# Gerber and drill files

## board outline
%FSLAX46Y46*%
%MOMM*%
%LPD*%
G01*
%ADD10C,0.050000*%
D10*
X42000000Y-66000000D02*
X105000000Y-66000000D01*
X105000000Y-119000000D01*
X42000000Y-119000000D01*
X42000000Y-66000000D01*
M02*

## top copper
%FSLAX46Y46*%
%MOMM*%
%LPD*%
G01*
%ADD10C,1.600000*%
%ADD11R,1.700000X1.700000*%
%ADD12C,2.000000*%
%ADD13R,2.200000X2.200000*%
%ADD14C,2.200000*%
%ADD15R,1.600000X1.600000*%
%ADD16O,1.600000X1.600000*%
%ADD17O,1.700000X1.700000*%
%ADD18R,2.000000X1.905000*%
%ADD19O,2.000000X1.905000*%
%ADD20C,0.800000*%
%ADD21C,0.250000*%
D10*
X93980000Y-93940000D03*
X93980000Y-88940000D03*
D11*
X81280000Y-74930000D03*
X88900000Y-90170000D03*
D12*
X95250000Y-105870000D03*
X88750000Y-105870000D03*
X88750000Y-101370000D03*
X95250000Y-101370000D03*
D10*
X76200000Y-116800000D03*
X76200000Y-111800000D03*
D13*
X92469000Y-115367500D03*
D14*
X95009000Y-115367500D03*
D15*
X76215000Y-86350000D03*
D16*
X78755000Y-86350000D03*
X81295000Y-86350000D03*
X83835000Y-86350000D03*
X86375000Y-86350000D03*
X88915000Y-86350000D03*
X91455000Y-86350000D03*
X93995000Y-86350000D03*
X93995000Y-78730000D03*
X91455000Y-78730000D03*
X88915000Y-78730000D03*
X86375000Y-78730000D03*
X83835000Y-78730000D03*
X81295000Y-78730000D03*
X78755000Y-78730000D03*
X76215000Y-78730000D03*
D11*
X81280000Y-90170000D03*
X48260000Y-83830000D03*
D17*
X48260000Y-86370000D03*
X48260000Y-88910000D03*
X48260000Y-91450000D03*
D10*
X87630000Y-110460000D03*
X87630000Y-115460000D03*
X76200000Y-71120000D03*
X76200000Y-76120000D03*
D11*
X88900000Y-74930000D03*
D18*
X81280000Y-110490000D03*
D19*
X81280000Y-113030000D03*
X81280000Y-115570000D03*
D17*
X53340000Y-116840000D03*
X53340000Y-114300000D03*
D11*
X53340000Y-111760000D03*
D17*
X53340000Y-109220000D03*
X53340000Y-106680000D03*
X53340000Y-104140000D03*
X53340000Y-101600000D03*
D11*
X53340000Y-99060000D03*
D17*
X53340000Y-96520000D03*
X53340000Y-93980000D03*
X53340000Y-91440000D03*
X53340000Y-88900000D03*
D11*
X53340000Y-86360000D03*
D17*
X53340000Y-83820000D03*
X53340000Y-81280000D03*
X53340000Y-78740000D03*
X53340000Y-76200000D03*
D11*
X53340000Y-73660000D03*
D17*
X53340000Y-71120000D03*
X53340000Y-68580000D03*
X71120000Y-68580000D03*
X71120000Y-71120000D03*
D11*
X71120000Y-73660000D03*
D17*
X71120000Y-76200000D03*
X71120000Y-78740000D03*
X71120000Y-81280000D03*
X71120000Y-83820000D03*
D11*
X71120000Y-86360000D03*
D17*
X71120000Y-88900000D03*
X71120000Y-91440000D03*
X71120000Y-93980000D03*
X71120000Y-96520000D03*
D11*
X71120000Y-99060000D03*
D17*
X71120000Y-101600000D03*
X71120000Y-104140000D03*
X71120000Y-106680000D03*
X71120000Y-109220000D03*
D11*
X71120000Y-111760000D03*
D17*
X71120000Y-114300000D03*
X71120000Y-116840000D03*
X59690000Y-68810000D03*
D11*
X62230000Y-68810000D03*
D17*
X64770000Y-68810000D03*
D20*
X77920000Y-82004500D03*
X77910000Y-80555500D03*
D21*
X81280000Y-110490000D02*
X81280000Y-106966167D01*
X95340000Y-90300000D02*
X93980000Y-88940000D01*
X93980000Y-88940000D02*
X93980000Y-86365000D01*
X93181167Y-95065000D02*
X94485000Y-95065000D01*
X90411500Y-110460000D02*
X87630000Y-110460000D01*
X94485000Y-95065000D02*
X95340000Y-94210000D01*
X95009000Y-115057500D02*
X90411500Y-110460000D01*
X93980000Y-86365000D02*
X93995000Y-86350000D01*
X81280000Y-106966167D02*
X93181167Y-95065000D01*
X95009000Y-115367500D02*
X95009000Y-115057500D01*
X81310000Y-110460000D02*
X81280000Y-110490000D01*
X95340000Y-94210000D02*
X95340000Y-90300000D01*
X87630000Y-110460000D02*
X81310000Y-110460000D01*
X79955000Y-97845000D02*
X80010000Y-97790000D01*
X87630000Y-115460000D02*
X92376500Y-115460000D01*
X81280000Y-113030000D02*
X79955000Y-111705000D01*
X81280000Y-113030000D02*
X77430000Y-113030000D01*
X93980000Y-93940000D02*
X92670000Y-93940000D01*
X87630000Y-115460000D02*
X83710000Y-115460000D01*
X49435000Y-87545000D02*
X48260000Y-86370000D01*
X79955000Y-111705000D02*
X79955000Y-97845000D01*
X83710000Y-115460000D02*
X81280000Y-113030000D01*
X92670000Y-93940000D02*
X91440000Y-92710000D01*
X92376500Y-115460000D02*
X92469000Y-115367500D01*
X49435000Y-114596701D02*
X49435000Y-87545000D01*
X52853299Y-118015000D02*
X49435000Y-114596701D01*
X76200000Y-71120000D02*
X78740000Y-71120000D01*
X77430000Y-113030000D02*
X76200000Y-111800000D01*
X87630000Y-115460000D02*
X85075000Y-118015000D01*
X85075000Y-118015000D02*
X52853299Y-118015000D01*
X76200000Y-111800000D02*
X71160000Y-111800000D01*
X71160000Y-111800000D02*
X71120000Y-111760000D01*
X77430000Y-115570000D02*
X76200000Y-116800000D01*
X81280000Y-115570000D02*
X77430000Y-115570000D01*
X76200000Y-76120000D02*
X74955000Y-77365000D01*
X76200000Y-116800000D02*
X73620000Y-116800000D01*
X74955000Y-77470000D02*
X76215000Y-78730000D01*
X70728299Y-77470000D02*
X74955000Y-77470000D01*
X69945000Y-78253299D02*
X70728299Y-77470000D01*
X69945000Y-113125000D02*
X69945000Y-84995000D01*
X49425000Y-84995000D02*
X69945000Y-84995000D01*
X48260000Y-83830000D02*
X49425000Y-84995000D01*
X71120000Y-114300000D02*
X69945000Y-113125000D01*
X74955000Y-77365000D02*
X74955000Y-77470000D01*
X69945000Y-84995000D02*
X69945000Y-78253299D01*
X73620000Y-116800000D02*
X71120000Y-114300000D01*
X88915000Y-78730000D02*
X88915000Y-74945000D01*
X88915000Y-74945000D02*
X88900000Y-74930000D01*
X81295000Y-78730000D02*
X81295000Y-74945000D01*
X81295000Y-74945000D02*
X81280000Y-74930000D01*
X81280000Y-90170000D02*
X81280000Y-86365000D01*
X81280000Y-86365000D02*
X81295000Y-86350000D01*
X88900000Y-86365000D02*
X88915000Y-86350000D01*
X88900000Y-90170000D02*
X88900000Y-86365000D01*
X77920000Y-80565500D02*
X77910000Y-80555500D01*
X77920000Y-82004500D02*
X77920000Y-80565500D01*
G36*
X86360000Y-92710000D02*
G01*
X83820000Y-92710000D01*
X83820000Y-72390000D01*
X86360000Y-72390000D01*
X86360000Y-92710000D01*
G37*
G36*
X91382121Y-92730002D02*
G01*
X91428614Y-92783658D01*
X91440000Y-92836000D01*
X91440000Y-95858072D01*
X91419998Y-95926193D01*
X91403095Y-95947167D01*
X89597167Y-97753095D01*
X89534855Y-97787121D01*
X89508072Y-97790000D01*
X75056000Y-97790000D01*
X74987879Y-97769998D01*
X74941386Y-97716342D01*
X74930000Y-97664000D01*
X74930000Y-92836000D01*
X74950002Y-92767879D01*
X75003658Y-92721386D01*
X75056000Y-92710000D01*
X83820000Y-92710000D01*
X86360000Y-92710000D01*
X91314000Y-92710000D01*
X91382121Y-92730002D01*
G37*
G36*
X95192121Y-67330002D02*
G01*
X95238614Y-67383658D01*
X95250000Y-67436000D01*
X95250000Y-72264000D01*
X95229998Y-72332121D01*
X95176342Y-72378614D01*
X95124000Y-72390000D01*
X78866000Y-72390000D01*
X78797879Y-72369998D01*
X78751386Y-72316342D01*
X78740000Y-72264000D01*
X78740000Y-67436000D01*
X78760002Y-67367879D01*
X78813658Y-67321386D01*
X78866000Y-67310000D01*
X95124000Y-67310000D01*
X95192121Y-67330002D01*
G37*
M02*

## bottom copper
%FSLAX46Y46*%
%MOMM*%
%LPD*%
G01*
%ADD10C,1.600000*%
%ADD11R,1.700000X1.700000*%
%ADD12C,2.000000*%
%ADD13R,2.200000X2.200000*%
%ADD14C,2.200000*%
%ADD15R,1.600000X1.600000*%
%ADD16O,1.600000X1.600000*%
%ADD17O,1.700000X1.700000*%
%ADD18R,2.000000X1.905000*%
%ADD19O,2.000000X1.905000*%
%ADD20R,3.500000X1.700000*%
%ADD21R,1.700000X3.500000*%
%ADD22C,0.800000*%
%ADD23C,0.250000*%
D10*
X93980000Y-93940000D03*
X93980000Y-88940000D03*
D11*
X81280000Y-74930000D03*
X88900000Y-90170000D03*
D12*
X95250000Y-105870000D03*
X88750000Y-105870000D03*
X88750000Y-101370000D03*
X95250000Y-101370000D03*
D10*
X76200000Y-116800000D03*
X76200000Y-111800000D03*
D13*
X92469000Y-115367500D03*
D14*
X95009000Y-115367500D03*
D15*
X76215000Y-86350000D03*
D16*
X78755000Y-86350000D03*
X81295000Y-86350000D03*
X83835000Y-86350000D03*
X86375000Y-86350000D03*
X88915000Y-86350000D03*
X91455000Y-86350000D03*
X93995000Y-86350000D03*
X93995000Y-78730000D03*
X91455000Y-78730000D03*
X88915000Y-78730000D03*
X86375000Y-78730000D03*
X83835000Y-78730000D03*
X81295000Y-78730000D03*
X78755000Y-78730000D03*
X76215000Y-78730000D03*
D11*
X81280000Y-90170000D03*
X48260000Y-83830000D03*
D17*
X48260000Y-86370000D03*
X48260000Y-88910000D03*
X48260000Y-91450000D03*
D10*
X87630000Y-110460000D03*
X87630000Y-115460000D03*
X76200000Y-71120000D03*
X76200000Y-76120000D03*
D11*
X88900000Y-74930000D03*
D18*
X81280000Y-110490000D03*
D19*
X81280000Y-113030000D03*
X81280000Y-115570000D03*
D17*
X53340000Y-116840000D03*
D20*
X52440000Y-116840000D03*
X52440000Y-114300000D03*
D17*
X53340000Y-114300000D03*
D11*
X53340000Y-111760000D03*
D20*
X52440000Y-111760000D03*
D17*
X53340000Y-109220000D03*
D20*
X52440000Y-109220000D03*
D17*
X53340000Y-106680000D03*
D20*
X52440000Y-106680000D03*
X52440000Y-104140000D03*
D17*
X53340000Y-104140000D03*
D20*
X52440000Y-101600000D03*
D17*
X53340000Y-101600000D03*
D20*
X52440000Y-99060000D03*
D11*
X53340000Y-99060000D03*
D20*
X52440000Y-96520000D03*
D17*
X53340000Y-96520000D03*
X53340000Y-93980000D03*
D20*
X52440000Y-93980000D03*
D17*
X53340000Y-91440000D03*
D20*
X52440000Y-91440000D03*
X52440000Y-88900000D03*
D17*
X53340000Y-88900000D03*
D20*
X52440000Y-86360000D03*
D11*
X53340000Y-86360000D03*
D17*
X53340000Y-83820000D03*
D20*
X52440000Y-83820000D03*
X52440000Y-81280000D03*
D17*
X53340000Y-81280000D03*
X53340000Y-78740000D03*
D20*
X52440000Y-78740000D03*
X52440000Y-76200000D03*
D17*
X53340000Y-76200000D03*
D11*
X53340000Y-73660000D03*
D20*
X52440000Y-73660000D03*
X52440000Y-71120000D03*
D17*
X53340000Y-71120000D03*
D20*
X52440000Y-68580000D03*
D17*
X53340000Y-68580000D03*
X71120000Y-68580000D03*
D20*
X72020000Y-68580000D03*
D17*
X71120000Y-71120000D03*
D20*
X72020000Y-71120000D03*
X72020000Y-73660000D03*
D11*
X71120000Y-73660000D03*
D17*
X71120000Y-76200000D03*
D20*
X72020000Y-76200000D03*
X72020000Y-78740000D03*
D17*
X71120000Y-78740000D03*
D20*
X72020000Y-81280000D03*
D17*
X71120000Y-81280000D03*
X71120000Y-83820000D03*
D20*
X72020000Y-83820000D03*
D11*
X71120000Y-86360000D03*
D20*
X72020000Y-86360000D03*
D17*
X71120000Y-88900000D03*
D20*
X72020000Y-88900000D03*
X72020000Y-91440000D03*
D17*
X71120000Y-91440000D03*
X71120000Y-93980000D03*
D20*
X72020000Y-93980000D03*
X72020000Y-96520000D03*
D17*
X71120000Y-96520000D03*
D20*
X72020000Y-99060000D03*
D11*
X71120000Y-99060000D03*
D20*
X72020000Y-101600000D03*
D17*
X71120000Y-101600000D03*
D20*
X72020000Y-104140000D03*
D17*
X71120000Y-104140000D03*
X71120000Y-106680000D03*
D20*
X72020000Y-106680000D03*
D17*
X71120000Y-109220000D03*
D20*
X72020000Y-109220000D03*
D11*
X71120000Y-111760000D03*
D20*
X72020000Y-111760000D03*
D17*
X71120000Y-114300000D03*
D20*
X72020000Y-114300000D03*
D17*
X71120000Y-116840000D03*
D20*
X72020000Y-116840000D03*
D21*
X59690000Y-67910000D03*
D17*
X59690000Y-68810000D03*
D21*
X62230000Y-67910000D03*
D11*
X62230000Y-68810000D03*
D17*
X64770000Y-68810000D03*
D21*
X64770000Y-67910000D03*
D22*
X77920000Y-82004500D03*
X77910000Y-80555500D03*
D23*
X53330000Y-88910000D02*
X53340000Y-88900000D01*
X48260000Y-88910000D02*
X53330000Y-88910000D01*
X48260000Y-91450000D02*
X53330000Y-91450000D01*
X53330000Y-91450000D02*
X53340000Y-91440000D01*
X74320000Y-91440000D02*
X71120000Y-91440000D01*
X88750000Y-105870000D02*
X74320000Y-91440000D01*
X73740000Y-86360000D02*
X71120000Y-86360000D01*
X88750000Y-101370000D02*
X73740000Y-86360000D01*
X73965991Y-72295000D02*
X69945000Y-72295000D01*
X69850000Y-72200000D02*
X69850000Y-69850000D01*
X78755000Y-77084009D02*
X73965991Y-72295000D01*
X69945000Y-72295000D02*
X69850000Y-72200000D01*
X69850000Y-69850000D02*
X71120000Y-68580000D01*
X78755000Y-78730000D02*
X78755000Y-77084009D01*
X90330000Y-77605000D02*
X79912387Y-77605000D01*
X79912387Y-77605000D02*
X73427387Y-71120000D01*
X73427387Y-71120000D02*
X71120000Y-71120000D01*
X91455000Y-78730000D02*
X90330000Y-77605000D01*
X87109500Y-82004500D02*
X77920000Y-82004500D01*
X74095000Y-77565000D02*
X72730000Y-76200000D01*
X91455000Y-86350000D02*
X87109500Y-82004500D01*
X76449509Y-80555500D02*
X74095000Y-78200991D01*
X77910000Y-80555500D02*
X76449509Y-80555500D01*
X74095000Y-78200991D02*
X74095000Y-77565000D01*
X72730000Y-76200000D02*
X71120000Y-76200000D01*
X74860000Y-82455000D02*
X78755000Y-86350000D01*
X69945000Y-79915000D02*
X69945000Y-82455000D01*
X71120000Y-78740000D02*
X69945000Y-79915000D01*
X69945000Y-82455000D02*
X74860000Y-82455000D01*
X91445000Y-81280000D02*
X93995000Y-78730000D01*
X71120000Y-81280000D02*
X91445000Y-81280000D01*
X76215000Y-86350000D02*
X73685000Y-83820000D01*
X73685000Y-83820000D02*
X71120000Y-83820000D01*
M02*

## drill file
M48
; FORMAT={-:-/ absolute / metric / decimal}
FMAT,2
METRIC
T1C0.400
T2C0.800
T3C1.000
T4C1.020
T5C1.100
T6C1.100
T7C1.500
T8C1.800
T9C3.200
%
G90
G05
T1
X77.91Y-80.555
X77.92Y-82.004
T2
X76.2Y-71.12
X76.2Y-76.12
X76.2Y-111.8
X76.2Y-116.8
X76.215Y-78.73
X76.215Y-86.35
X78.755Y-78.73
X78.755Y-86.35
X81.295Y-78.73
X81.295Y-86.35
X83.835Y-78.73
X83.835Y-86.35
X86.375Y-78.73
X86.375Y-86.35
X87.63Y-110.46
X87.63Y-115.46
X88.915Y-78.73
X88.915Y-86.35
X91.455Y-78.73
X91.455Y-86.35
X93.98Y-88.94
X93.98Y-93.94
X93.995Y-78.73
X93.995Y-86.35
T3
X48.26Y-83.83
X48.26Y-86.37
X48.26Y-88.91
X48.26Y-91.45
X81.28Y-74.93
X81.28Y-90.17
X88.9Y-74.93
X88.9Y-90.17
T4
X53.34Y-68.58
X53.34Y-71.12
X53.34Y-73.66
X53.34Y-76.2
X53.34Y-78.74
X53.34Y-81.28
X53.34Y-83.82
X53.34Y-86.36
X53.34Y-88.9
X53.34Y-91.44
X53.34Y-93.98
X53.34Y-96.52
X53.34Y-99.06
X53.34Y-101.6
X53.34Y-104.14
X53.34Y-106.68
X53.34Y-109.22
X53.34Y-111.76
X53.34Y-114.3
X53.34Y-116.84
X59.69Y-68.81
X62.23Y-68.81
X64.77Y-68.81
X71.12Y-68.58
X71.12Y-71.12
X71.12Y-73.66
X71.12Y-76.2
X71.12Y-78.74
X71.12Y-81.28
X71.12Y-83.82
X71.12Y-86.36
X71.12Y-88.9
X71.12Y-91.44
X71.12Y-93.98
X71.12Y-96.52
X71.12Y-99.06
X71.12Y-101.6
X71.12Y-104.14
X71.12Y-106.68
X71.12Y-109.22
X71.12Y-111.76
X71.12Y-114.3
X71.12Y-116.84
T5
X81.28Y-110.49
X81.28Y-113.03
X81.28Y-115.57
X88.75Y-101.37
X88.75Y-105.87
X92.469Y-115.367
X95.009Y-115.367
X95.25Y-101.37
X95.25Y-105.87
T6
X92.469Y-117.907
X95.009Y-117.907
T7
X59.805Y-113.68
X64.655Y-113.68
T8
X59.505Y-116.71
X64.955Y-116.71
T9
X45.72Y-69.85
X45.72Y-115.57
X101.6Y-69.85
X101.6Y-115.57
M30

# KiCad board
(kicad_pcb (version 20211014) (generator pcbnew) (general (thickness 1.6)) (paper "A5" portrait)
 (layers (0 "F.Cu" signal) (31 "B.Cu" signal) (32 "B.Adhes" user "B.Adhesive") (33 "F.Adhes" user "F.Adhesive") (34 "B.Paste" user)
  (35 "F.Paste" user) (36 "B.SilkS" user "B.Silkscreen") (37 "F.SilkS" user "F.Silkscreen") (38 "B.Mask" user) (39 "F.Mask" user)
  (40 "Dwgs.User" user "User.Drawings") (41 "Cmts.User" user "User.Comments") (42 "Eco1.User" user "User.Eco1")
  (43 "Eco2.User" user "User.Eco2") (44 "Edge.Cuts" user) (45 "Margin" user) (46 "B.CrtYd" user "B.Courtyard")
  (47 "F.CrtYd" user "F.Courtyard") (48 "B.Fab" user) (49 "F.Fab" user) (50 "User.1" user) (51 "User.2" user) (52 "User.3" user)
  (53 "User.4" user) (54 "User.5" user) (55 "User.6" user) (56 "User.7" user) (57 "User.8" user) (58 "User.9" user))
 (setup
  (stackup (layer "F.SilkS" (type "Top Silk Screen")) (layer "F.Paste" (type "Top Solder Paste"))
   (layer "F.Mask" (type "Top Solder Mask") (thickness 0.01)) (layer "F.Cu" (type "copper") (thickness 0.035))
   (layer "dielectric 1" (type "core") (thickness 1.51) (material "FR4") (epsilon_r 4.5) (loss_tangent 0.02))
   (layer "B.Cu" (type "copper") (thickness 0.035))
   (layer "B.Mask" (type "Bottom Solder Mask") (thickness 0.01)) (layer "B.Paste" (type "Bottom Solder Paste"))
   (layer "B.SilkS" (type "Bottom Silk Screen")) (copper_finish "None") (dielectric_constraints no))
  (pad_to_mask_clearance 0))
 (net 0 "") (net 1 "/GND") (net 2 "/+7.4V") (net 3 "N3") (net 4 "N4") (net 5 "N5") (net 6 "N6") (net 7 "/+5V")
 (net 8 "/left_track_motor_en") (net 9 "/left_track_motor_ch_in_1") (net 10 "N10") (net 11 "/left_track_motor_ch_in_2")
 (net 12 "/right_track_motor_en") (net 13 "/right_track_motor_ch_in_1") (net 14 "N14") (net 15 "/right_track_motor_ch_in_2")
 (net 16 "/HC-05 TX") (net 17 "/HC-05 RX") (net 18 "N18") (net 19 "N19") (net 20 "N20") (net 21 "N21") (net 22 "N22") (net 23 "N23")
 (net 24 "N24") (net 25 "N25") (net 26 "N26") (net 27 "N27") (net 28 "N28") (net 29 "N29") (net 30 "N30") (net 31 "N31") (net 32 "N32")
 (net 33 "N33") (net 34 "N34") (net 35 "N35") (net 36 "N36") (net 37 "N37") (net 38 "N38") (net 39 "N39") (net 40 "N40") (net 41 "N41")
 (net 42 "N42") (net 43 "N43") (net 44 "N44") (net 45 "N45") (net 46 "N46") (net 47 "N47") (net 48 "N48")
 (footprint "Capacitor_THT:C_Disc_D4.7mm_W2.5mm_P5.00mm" (layer "F.Cu") (at 93.98 93.94 90)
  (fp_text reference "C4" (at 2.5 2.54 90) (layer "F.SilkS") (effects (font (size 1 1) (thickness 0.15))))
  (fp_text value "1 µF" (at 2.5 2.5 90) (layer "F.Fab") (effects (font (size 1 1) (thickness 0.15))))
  (pad "1" thru_hole circle (at 0 0 90) (size 1.6 1.6) (drill 0.8) (layers *.Cu *.Mask) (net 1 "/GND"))
  (pad "2" thru_hole circle (at 5 0 90) (size 1.6 1.6) (drill 0.8) (layers *.Cu *.Mask) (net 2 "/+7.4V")))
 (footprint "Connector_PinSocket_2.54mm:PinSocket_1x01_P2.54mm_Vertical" (layer "F.Cu") (at 81.28 74.93 90)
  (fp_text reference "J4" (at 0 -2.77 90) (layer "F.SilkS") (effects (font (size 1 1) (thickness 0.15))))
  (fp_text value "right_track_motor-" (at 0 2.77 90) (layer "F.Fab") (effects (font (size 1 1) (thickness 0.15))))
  (pad "1" thru_hole rect (at 0 0 90) (size 1.7 1.7) (drill 1) (layers *.Cu *.Mask) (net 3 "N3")))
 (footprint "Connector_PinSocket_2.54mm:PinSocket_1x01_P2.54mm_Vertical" (layer "F.Cu") (at 88.9 90.17 90)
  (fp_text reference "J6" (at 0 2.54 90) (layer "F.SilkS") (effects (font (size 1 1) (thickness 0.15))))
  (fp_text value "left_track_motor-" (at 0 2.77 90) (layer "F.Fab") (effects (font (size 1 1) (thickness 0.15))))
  (pad "1" thru_hole rect (at 0 0 90) (size 1.7 1.7) (drill 1) (layers *.Cu *.Mask) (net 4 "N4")))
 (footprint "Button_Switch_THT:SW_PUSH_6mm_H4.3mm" (layer "F.Cu") (at 95.25 105.87 180)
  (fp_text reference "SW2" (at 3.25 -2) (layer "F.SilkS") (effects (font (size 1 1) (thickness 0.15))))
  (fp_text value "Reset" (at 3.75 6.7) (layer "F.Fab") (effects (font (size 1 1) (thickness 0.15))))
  (pad "1" thru_hole circle (at 0 0 270) (size 2 2) (drill 1.1) (layers *.Cu *.Mask) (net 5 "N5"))
  (pad "1" thru_hole circle (at 6.5 0 270) (size 2 2) (drill 1.1) (layers *.Cu *.Mask) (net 5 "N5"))
  (pad "2" thru_hole circle (at 6.5 4.5 270) (size 2 2) (drill 1.1) (layers *.Cu *.Mask) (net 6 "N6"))
  (pad "2" thru_hole circle (at 0 4.5 270) (size 2 2) (drill 1.1) (layers *.Cu *.Mask) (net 6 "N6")))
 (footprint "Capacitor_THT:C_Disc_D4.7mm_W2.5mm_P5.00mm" (layer "F.Cu") (at 76.2 116.8 90)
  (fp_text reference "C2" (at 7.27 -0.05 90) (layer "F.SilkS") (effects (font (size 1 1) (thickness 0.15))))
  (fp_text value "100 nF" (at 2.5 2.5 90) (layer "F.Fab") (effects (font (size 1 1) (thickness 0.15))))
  (pad "1" thru_hole circle (at 0 0 90) (size 1.6 1.6) (drill 0.8) (layers *.Cu *.Mask) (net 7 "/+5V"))
  (pad "2" thru_hole circle (at 5 0 90) (size 1.6 1.6) (drill 0.8) (layers *.Cu *.Mask) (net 1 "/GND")))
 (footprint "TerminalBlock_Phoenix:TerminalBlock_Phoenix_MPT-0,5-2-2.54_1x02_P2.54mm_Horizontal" (layer "F.Cu") (at 92.469 115.3675)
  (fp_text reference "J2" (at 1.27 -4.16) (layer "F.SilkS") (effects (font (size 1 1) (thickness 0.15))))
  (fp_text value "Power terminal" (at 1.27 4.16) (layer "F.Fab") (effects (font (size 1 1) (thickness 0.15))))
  (pad "" np_thru_hole circle (at 0 2.54) (size 1.1 1.1) (drill 1.1) (layers *.Cu *.Mask))
  (pad "" np_thru_hole circle (at 2.54 2.54) (size 1.1 1.1) (drill 1.1) (layers *.Cu *.Mask))
  (pad "1" thru_hole rect (at 0 0) (size 2.2 2.2) (drill 1.1) (layers *.Cu *.Mask) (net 1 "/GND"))
  (pad "2" thru_hole circle (at 2.54 0) (size 2.2 2.2) (drill 1.1) (layers *.Cu *.Mask) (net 2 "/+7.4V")))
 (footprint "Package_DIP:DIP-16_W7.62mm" (layer "F.Cu") (at 76.215 86.35 90)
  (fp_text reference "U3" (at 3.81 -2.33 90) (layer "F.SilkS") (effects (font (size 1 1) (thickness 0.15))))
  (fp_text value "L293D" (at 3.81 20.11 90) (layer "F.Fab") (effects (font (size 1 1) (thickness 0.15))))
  (pad "1" thru_hole rect (at 0 0 90) (size 1.6 1.6) (drill 0.8) (layers *.Cu *.Mask) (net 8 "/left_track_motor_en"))
  (pad "2" thru_hole oval (at 0 2.54 90) (size 1.6 1.6) (drill 0.8) (layers *.Cu *.Mask) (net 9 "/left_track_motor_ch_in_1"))
  (pad "3" thru_hole oval (at 0 5.08 90) (size 1.6 1.6) (drill 0.8) (layers *.Cu *.Mask) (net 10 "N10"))
  (pad "4" thru_hole oval (at 0 7.62 90) (size 1.6 1.6) (drill 0.8) (layers *.Cu *.Mask) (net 1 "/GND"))
  (pad "5" thru_hole oval (at 0 10.16 90) (size 1.6 1.6) (drill 0.8) (layers *.Cu *.Mask) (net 1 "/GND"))
  (pad "6" thru_hole oval (at 0 12.7 90) (size 1.6 1.6) (drill 0.8) (layers *.Cu *.Mask) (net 4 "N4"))
  (pad "7" thru_hole oval (at 0 15.24 90) (size 1.6 1.6) (drill 0.8) (layers *.Cu *.Mask) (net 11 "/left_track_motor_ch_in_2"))
  (pad "8" thru_hole oval (at 0 17.78 90) (size 1.6 1.6) (drill 0.8) (layers *.Cu *.Mask) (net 2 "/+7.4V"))
  (pad "9" thru_hole oval (at 7.62 17.78 90) (size 1.6 1.6) (drill 0.8) (layers *.Cu *.Mask) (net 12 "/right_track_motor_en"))
  (pad "10" thru_hole oval (at 7.62 15.24 90) (size 1.6 1.6) (drill 0.8) (layers *.Cu *.Mask) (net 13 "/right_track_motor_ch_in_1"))
  (pad "11" thru_hole oval (at 7.62 12.7 90) (size 1.6 1.6) (drill 0.8) (layers *.Cu *.Mask) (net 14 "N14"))
  (pad "12" thru_hole oval (at 7.62 10.16 90) (size 1.6 1.6) (drill 0.8) (layers *.Cu *.Mask) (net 1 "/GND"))
  (pad "13" thru_hole oval (at 7.62 7.62 90) (size 1.6 1.6) (drill 0.8) (layers *.Cu *.Mask) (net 1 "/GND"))
  (pad "14" thru_hole oval (at 7.62 5.08 90) (size 1.6 1.6) (drill 0.8) (layers *.Cu *.Mask) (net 3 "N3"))
  (pad "15" thru_hole oval (at 7.62 2.54 90) (size 1.6 1.6) (drill 0.8) (layers *.Cu *.Mask) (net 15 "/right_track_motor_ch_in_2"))
  (pad "16" thru_hole oval (at 7.62 0 90) (size 1.6 1.6) (drill 0.8) (layers *.Cu *.Mask) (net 7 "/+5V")))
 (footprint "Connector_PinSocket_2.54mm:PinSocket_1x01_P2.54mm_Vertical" (layer "F.Cu") (at 81.28 90.17 90)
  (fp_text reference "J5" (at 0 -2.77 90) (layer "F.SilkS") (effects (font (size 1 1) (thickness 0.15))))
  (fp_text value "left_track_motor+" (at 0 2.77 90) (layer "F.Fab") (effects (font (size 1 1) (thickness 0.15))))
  (pad "1" thru_hole rect (at 0 0 90) (size 1.7 1.7) (drill 1) (layers *.Cu *.Mask) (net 10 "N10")))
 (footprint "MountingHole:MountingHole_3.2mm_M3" (layer "F.Cu") (at 101.6 115.57)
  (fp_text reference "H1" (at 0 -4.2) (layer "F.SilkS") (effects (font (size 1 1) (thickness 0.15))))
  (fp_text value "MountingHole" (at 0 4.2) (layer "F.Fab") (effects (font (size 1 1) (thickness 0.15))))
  (pad "" np_thru_hole circle (at 0 0) (size 3.2 3.2) (drill 3.2) (layers *.Cu *.Mask)))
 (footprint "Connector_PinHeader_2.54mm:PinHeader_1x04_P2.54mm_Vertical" (layer "F.Cu") (at 48.26 83.83)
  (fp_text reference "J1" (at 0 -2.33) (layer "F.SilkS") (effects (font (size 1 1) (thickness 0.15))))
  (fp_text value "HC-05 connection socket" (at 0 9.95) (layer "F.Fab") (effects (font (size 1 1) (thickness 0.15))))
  (pad "1" thru_hole rect (at 0 0) (size 1.7 1.7) (drill 1) (layers *.Cu *.Mask) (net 7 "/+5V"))
  (pad "2" thru_hole oval (at 0 2.54) (size 1.7 1.7) (drill 1) (layers *.Cu *.Mask) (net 1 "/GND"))
  (pad "3" thru_hole oval (at 0 5.08) (size 1.7 1.7) (drill 1) (layers *.Cu *.Mask) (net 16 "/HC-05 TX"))
  (pad "4" thru_hole oval (at 0 7.62) (size 1.7 1.7) (drill 1) (layers *.Cu *.Mask) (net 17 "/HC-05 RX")))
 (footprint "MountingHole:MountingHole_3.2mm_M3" (layer "F.Cu") (at 101.6 69.85)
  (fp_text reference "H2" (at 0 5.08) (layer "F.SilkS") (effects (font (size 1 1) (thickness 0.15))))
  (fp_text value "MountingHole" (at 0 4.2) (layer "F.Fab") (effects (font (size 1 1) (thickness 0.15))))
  (pad "" np_thru_hole circle (at 0 0) (size 3.2 3.2) (drill 3.2) (layers *.Cu *.Mask)))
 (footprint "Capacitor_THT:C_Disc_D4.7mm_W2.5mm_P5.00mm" (layer "F.Cu") (at 87.63 110.46 -90)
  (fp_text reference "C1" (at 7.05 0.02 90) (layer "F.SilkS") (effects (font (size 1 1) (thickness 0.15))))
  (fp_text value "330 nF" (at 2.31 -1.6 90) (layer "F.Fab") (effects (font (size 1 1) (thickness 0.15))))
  (pad "1" thru_hole circle (at 0 0 270) (size 1.6 1.6) (drill 0.8) (layers *.Cu *.Mask) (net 2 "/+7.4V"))
  (pad "2" thru_hole circle (at 5 0 270) (size 1.6 1.6) (drill 0.8) (layers *.Cu *.Mask) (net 1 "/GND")))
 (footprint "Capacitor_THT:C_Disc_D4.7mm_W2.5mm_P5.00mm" (layer "F.Cu") (at 76.2 71.12 -90)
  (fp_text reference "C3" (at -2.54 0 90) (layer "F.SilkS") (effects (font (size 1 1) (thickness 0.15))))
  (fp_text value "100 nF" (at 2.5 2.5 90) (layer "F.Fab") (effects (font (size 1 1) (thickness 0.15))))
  (pad "1" thru_hole circle (at 0 0 270) (size 1.6 1.6) (drill 0.8) (layers *.Cu *.Mask) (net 1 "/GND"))
  (pad "2" thru_hole circle (at 5 0 270) (size 1.6 1.6) (drill 0.8) (layers *.Cu *.Mask) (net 7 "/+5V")))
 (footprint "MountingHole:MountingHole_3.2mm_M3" (layer "F.Cu") (at 45.72 69.85)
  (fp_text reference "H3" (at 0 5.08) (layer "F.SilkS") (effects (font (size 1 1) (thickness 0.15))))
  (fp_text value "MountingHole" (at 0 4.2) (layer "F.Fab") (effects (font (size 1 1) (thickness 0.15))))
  (pad "" np_thru_hole circle (at 0 0) (size 3.2 3.2) (drill 3.2) (layers *.Cu *.Mask)))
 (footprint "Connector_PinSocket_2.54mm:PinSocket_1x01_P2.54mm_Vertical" (layer "F.Cu") (at 88.9 74.93 90)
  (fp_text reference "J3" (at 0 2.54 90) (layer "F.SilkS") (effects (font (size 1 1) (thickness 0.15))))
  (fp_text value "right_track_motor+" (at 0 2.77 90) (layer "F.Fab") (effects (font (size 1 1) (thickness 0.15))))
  (pad "1" thru_hole rect (at 0 0 90) (size 1.7 1.7) (drill 1) (layers *.Cu *.Mask) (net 14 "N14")))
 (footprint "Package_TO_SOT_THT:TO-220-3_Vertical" (layer "F.Cu") (at 81.28 110.49 -90)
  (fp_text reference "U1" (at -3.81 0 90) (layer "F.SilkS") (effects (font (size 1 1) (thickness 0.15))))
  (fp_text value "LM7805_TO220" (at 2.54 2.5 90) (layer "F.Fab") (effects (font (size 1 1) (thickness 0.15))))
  (pad "1" thru_hole rect (at 0 0 270) (size 1.905 2) (drill 1.1) (layers *.Cu *.Mask) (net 2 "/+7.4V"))
  (pad "2" thru_hole oval (at 2.54 0 270) (size 1.905 2) (drill 1.1) (layers *.Cu *.Mask) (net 1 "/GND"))
  (pad "3" thru_hole oval (at 5.08 0 270) (size 1.905 2) (drill 1.1) (layers *.Cu *.Mask) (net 7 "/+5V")))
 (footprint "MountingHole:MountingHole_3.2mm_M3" (layer "F.Cu") (at 45.72 115.57)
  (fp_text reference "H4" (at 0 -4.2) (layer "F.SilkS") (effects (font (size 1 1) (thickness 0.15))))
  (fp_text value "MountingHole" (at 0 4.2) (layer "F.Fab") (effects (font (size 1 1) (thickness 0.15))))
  (pad "" np_thru_hole circle (at 0 0) (size 3.2 3.2) (drill 3.2) (layers *.Cu *.Mask)))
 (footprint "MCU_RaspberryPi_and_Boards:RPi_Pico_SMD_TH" (layer "B.Cu") (at 62.23 92.71)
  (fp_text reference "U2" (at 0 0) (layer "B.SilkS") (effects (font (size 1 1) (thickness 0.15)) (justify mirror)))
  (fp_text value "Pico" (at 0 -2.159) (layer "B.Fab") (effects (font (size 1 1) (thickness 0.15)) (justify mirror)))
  (pad "" np_thru_hole oval (at -2.725 24) (size 1.8 1.8) (drill 1.8) (layers *.Cu *.Mask))
  (pad "" np_thru_hole oval (at -2.425 20.97) (size 1.5 1.5) (drill 1.5) (layers *.Cu *.Mask))
  (pad "" np_thru_hole oval (at 2.425 20.97) (size 1.5 1.5) (drill 1.5) (layers *.Cu *.Mask))
  (pad "" np_thru_hole oval (at 2.725 24) (size 1.8 1.8) (drill 1.8) (layers *.Cu *.Mask))
  (pad "1" thru_hole oval (at -8.89 24.13) (size 1.7 1.7) (drill 1.02) (layers *.Cu *.Mask) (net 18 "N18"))
  (pad "1" smd rect (at -8.89 24.13) (size 3.5 1.7) (drill (offset -0.9 0)) (layers "B.Cu" "B.Mask") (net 18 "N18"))
  (pad "2" smd rect (at -8.89 21.59) (size 3.5 1.7) (drill (offset -0.9 0)) (layers "B.Cu" "B.Mask") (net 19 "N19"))
  (pad "2" thru_hole oval (at -8.89 21.59) (size 1.7 1.7) (drill 1.02) (layers *.Cu *.Mask) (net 19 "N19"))
  (pad "3" thru_hole rect (at -8.89 19.05) (size 1.7 1.7) (drill 1.02) (layers *.Cu *.Mask) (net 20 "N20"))
  (pad "3" smd rect (at -8.89 19.05) (size 3.5 1.7) (drill (offset -0.9 0)) (layers "B.Cu" "B.Mask") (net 20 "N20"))
  (pad "4" thru_hole oval (at -8.89 16.51) (size 1.7 1.7) (drill 1.02) (layers *.Cu *.Mask) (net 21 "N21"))
  (pad "4" smd rect (at -8.89 16.51) (size 3.5 1.7) (drill (offset -0.9 0)) (layers "B.Cu" "B.Mask") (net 21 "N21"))
  (pad "5" thru_hole oval (at -8.89 13.97) (size 1.7 1.7) (drill 1.02) (layers *.Cu *.Mask) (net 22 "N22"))
  (pad "5" smd rect (at -8.89 13.97) (size 3.5 1.7) (drill (offset -0.9 0)) (layers "B.Cu" "B.Mask") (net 22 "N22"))
  (pad "6" smd rect (at -8.89 11.43) (size 3.5 1.7) (drill (offset -0.9 0)) (layers "B.Cu" "B.Mask") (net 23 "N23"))
  (pad "6" thru_hole oval (at -8.89 11.43) (size 1.7 1.7) (drill 1.02) (layers *.Cu *.Mask) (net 23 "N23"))
  (pad "7" smd rect (at -8.89 8.89) (size 3.5 1.7) (drill (offset -0.9 0)) (layers "B.Cu" "B.Mask") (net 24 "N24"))
  (pad "7" thru_hole oval (at -8.89 8.89) (size 1.7 1.7) (drill 1.02) (layers *.Cu *.Mask) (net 24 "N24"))
  (pad "8" smd rect (at -8.89 6.35) (size 3.5 1.7) (drill (offset -0.9 0)) (layers "B.Cu" "B.Mask") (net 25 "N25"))
  (pad "8" thru_hole rect (at -8.89 6.35) (size 1.7 1.7) (drill 1.02) (layers *.Cu *.Mask) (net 25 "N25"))
  (pad "9" smd rect (at -8.89 3.81) (size 3.5 1.7) (drill (offset -0.9 0)) (layers "B.Cu" "B.Mask") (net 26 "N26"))
  (pad "9" thru_hole oval (at -8.89 3.81) (size 1.7 1.7) (drill 1.02) (layers *.Cu *.Mask) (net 26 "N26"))
  (pad "10" thru_hole oval (at -8.89 1.27) (size 1.7 1.7) (drill 1.02) (layers *.Cu *.Mask) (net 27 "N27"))
  (pad "10" smd rect (at -8.89 1.27) (size 3.5 1.7) (drill (offset -0.9 0)) (layers "B.Cu" "B.Mask") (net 27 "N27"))
  (pad "11" thru_hole oval (at -8.89 -1.27) (size 1.7 1.7) (drill 1.02) (layers *.Cu *.Mask) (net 17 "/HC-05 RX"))
  (pad "11" smd rect (at -8.89 -1.27) (size 3.5 1.7) (drill (offset -0.9 0)) (layers "B.Cu" "B.Mask") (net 17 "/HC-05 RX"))
  (pad "12" smd rect (at -8.89 -3.81) (size 3.5 1.7) (drill (offset -0.9 0)) (layers "B.Cu" "B.Mask") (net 16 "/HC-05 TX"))
  (pad "12" thru_hole oval (at -8.89 -3.81) (size 1.7 1.7) (drill 1.02) (layers *.Cu *.Mask) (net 16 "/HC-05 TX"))
  (pad "13" smd rect (at -8.89 -6.35) (size 3.5 1.7) (drill (offset -0.9 0)) (layers "B.Cu" "B.Mask") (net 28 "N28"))
  (pad "13" thru_hole rect (at -8.89 -6.35) (size 1.7 1.7) (drill 1.02) (layers *.Cu *.Mask) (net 28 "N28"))
  (pad "14" thru_hole oval (at -8.89 -8.89) (size 1.7 1.7) (drill 1.02) (layers *.Cu *.Mask) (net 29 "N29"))
  (pad "14" smd rect (at -8.89 -8.89) (size 3.5 1.7) (drill (offset -0.9 0)) (layers "B.Cu" "B.Mask") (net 29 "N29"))
  (pad "15" smd rect (at -8.89 -11.43) (size 3.5 1.7) (drill (offset -0.9 0)) (layers "B.Cu" "B.Mask") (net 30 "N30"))
  (pad "15" thru_hole oval (at -8.89 -11.43) (size 1.7 1.7) (drill 1.02) (layers *.Cu *.Mask) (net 30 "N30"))
  (pad "16" thru_hole oval (at -8.89 -13.97) (size 1.7 1.7) (drill 1.02) (layers *.Cu *.Mask) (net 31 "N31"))
  (pad "16" smd rect (at -8.89 -13.97) (size 3.5 1.7) (drill (offset -0.9 0)) (layers "B.Cu" "B.Mask") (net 31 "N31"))
  (pad "17" smd rect (at -8.89 -16.51) (size 3.5 1.7) (drill (offset -0.9 0)) (layers "B.Cu" "B.Mask") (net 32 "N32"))
  (pad "17" thru_hole oval (at -8.89 -16.51) (size 1.7 1.7) (drill 1.02) (layers *.Cu *.Mask) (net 32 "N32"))
  (pad "18" thru_hole rect (at -8.89 -19.05) (size 1.7 1.7) (drill 1.02) (layers *.Cu *.Mask) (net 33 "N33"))
  (pad "18" smd rect (at -8.89 -19.05) (size 3.5 1.7) (drill (offset -0.9 0)) (layers "B.Cu" "B.Mask") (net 33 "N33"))
  (pad "19" smd rect (at -8.89 -21.59) (size 3.5 1.7) (drill (offset -0.9 0)) (layers "B.Cu" "B.Mask") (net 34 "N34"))
  (pad "19" thru_hole oval (at -8.89 -21.59) (size 1.7 1.7) (drill 1.02) (layers *.Cu *.Mask) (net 34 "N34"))
  (pad "20" smd rect (at -8.89 -24.13) (size 3.5 1.7) (drill (offset -0.9 0)) (layers "B.Cu" "B.Mask") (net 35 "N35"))
  (pad "20" thru_hole oval (at -8.89 -24.13) (size 1.7 1.7) (drill 1.02) (layers *.Cu *.Mask) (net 35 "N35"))
  (pad "21" thru_hole oval (at 8.89 -24.13) (size 1.7 1.7) (drill 1.02) (layers *.Cu *.Mask) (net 15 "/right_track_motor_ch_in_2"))
  (pad "21" smd rect (at 8.89 -24.13) (size 3.5 1.7) (drill (offset 0.9 0)) (layers "B.Cu" "B.Mask") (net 15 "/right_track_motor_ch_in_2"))
  (pad "22" thru_hole oval (at 8.89 -21.59) (size 1.7 1.7) (drill 1.02) (layers *.Cu *.Mask) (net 13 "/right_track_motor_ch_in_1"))
  (pad "22" smd rect (at 8.89 -21.59) (size 3.5 1.7) (drill (offset 0.9 0)) (layers "B.Cu" "B.Mask") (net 13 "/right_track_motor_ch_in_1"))
  (pad "23" smd rect (at 8.89 -19.05) (size 3.5 1.7) (drill (offset 0.9 0)) (layers "B.Cu" "B.Mask") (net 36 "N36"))
  (pad "23" thru_hole rect (at 8.89 -19.05) (size 1.7 1.7) (drill 1.02) (layers *.Cu *.Mask) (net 36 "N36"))
  (pad "24" thru_hole oval (at 8.89 -16.51) (size 1.7 1.7) (drill 1.02) (layers *.Cu *.Mask) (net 11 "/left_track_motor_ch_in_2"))
  (pad "24" smd rect (at 8.89 -16.51) (size 3.5 1.7) (drill (offset 0.9 0)) (layers "B.Cu" "B.Mask") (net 11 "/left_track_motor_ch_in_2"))
  (pad "25" smd rect (at 8.89 -13.97) (size 3.5 1.7) (drill (offset 0.9 0)) (layers "B.Cu" "B.Mask") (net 9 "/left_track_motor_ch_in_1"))
  (pad "25" thru_hole oval (at 8.89 -13.97) (size 1.7 1.7) (drill 1.02) (layers *.Cu *.Mask) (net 9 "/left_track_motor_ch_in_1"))
  (pad "26" smd rect (at 8.89 -11.43) (size 3.5 1.7) (drill (offset 0.9 0)) (layers "B.Cu" "B.Mask") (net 12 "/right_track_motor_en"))
  (pad "26" thru_hole oval (at 8.89 -11.43) (size 1.7 1.7) (drill 1.02) (layers *.Cu *.Mask) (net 12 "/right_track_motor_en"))
  (pad "27" thru_hole oval (at 8.89 -8.89) (size 1.7 1.7) (drill 1.02) (layers *.Cu *.Mask) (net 8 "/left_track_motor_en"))
  (pad "27" smd rect (at 8.89 -8.89) (size 3.5 1.7) (drill (offset 0.9 0)) (layers "B.Cu" "B.Mask") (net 8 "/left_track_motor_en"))
  (pad "28" thru_hole rect (at 8.89 -6.35) (size 1.7 1.7) (drill 1.02) (layers *.Cu *.Mask) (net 6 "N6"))
  (pad "28" smd rect (at 8.89 -6.35) (size 3.5 1.7) (drill (offset 0.9 0)) (layers "B.Cu" "B.Mask") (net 6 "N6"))
  (pad "29" thru_hole oval (at 8.89 -3.81) (size 1.7 1.7) (drill 1.02) (layers *.Cu *.Mask) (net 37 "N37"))
  (pad "29" smd rect (at 8.89 -3.81) (size 3.5 1.7) (drill (offset 0.9 0)) (layers "B.Cu" "B.Mask") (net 37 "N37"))
  (pad "30" smd rect (at 8.89 -1.27) (size 3.5 1.7) (drill (offset 0.9 0)) (layers "B.Cu" "B.Mask") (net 5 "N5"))
  (pad "30" thru_hole oval (at 8.89 -1.27) (size 1.7 1.7) (drill 1.02) (layers *.Cu *.Mask) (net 5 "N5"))
  (pad "31" thru_hole oval (at 8.89 1.27) (size 1.7 1.7) (drill 1.02) (layers *.Cu *.Mask) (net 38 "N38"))
  (pad "31" smd rect (at 8.89 1.27) (size 3.5 1.7) (drill (offset 0.9 0)) (layers "B.Cu" "B.Mask") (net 38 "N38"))
  (pad "32" smd rect (at 8.89 3.81) (size 3.5 1.7) (drill (offset 0.9 0)) (layers "B.Cu" "B.Mask") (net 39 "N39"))
  (pad "32" thru_hole oval (at 8.89 3.81) (size 1.7 1.7) (drill 1.02) (layers *.Cu *.Mask) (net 39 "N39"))
  (pad "33" smd rect (at 8.89 6.35) (size 3.5 1.7) (drill (offset 0.9 0)) (layers "B.Cu" "B.Mask") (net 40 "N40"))
  (pad "33" thru_hole rect (at 8.89 6.35) (size 1.7 1.7) (drill 1.02) (layers *.Cu *.Mask) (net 40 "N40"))
  (pad "34" smd rect (at 8.89 8.89) (size 3.5 1.7) (drill (offset 0.9 0)) (layers "B.Cu" "B.Mask") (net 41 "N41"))
  (pad "34" thru_hole oval (at 8.89 8.89) (size 1.7 1.7) (drill 1.02) (layers *.Cu *.Mask) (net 41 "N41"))
  (pad "35" smd rect (at 8.89 11.43) (size 3.5 1.7) (drill (offset 0.9 0)) (layers "B.Cu" "B.Mask") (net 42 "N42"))
  (pad "35" thru_hole oval (at 8.89 11.43) (size 1.7 1.7) (drill 1.02) (layers *.Cu *.Mask) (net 42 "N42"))
  (pad "36" thru_hole oval (at 8.89 13.97) (size 1.7 1.7) (drill 1.02) (layers *.Cu *.Mask) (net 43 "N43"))
  (pad "36" smd rect (at 8.89 13.97) (size 3.5 1.7) (drill (offset 0.9 0)) (layers "B.Cu" "B.Mask") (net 43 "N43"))
  (pad "37" thru_hole oval (at 8.89 16.51) (size 1.7 1.7) (drill 1.02) (layers *.Cu *.Mask) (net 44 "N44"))
  (pad "37" smd rect (at 8.89 16.51) (size 3.5 1.7) (drill (offset 0.9 0)) (layers "B.Cu" "B.Mask") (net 44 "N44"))
  (pad "38" thru_hole rect (at 8.89 19.05) (size 1.7 1.7) (drill 1.02) (layers *.Cu *.Mask) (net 1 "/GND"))
  (pad "38" smd rect (at 8.89 19.05) (size 3.5 1.7) (drill (offset 0.9 0)) (layers "B.Cu" "B.Mask") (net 1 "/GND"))
  (pad "39" thru_hole oval (at 8.89 21.59) (size 1.7 1.7) (drill 1.02) (layers *.Cu *.Mask) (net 7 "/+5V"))
  (pad "39" smd rect (at 8.89 21.59) (size 3.5 1.7) (drill (offset 0.9 0)) (layers "B.Cu" "B.Mask") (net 7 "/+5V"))
  (pad "40" thru_hole oval (at 8.89 24.13) (size 1.7 1.7) (drill 1.02) (layers *.Cu *.Mask) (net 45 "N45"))
  (pad "40" smd rect (at 8.89 24.13) (size 3.5 1.7) (drill (offset 0.9 0)) (layers "B.Cu" "B.Mask") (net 45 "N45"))
  (pad "41" smd rect (at -2.54 -23.9 270) (size 3.5 1.7) (drill (offset -0.9 0)) (layers "B.Cu" "B.Mask") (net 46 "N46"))
  (pad "41" thru_hole oval (at -2.54 -23.9) (size 1.7 1.7) (drill 1.02) (layers *.Cu *.Mask) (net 46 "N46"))
  (pad "42" smd rect (at 0 -23.9 270) (size 3.5 1.7) (drill (offset -0.9 0)) (layers "B.Cu" "B.Mask") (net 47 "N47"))
  (pad "42" thru_hole rect (at 0 -23.9) (size 1.7 1.7) (drill 1.02) (layers *.Cu *.Mask) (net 47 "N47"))
  (pad "43" thru_hole oval (at 2.54 -23.9) (size 1.7 1.7) (drill 1.02) (layers *.Cu *.Mask) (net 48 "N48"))
  (pad "43" smd rect (at 2.54 -23.9 270) (size 3.5 1.7) (drill (offset -0.9 0)) (layers "B.Cu" "B.Mask") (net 48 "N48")))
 (gr_rect (start 42 66) (end 105 119) (layer "Edge.Cuts") (width 0.05) (fill none))
 (segment (start 81.28 110.49) (end 81.28 106.966167) (width 0.25) (layer "F.Cu") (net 2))
 (segment (start 95.34 90.3) (end 93.98 88.94) (width 0.25) (layer "F.Cu") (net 2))
 (segment (start 93.98 88.94) (end 93.98 86.365) (width 0.25) (layer "F.Cu") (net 2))
 (segment (start 93.181167 95.065) (end 94.485 95.065) (width 0.25) (layer "F.Cu") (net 2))
 (segment (start 90.4115 110.46) (end 87.63 110.46) (width 0.25) (layer "F.Cu") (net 2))
 (segment (start 94.485 95.065) (end 95.34 94.21) (width 0.25) (layer "F.Cu") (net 2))
 (segment (start 95.009 115.0575) (end 90.4115 110.46) (width 0.25) (layer "F.Cu") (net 2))
 (segment (start 93.98 86.365) (end 93.995 86.35) (width 0.25) (layer "F.Cu") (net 2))
 (segment (start 81.28 106.966167) (end 93.181167 95.065) (width 0.25) (layer "F.Cu") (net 2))
 (segment (start 95.009 115.3675) (end 95.009 115.0575) (width 0.25) (layer "F.Cu") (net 2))
 (segment (start 81.31 110.46) (end 81.28 110.49) (width 0.25) (layer "F.Cu") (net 2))
 (segment (start 95.34 94.21) (end 95.34 90.3) (width 0.25) (layer "F.Cu") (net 2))
 (segment (start 87.63 110.46) (end 81.31 110.46) (width 0.25) (layer "F.Cu") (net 2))
 (segment (start 79.955 97.845) (end 80.01 97.79) (width 0.25) (layer "F.Cu") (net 1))
 (segment (start 87.63 115.46) (end 92.3765 115.46) (width 0.25) (layer "F.Cu") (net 1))
 (segment (start 81.28 113.03) (end 79.955 111.705) (width 0.25) (layer "F.Cu") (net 1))
 (segment (start 81.28 113.03) (end 77.43 113.03) (width 0.25) (layer "F.Cu") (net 1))
 (segment (start 93.98 93.94) (end 92.67 93.94) (width 0.25) (layer "F.Cu") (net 1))
 (segment (start 87.63 115.46) (end 83.71 115.46) (width 0.25) (layer "F.Cu") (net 1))
 (segment (start 49.435 87.545) (end 48.26 86.37) (width 0.25) (layer "F.Cu") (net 1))
 (segment (start 79.955 111.705) (end 79.955 97.845) (width 0.25) (layer "F.Cu") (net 1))
 (segment (start 83.71 115.46) (end 81.28 113.03) (width 0.25) (layer "F.Cu") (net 1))
 (segment (start 92.67 93.94) (end 91.44 92.71) (width 0.25) (layer "F.Cu") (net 1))
 (segment (start 92.3765 115.46) (end 92.469 115.3675) (width 0.25) (layer "F.Cu") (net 1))
 (segment (start 49.435 114.596701) (end 49.435 87.545) (width 0.25) (layer "F.Cu") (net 1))
 (segment (start 52.853299 118.015) (end 49.435 114.596701) (width 0.25) (layer "F.Cu") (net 1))
 (segment (start 76.2 71.12) (end 78.74 71.12) (width 0.25) (layer "F.Cu") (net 1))
 (segment (start 77.43 113.03) (end 76.2 111.8) (width 0.25) (layer "F.Cu") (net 1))
 (segment (start 87.63 115.46) (end 85.075 118.015) (width 0.25) (layer "F.Cu") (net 1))
 (segment (start 85.075 118.015) (end 52.853299 118.015) (width 0.25) (layer "F.Cu") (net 1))
 (segment (start 76.2 111.8) (end 71.16 111.8) (width 0.25) (layer "F.Cu") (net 1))
 (segment (start 71.16 111.8) (end 71.12 111.76) (width 0.25) (layer "F.Cu") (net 1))
 (segment (start 77.43 115.57) (end 76.2 116.8) (width 0.25) (layer "F.Cu") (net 7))
 (segment (start 81.28 115.57) (end 77.43 115.57) (width 0.25) (layer "F.Cu") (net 7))
 (segment (start 76.2 76.12) (end 74.955 77.365) (width 0.25) (layer "F.Cu") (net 7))
 (segment (start 76.2 116.8) (end 73.62 116.8) (width 0.25) (layer "F.Cu") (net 7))
 (segment (start 74.955 77.47) (end 76.215 78.73) (width 0.25) (layer "F.Cu") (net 7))
 (segment (start 70.728299 77.47) (end 74.955 77.47) (width 0.25) (layer "F.Cu") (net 7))
 (segment (start 69.945 78.253299) (end 70.728299 77.47) (width 0.25) (layer "F.Cu") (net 7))
 (segment (start 69.945 113.125) (end 69.945 84.995) (width 0.25) (layer "F.Cu") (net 7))
 (segment (start 49.425 84.995) (end 69.945 84.995) (width 0.25) (layer "F.Cu") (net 7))
 (segment (start 48.26 83.83) (end 49.425 84.995) (width 0.25) (layer "F.Cu") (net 7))
 (segment (start 71.12 114.3) (end 69.945 113.125) (width 0.25) (layer "F.Cu") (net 7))
 (segment (start 74.955 77.365) (end 74.955 77.47) (width 0.25) (layer "F.Cu") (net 7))
 (segment (start 69.945 84.995) (end 69.945 78.253299) (width 0.25) (layer "F.Cu") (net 7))
 (segment (start 73.62 116.8) (end 71.12 114.3) (width 0.25) (layer "F.Cu") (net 7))
 (segment (start 53.33 88.91) (end 53.34 88.9) (width 0.25) (layer "B.Cu") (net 16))
 (segment (start 48.26 88.91) (end 53.33 88.91) (width 0.25) (layer "B.Cu") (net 16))
 (segment (start 48.26 91.45) (end 53.33 91.45) (width 0.25) (layer "B.Cu") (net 17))
 (segment (start 53.33 91.45) (end 53.34 91.44) (width 0.25) (layer "B.Cu") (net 17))
 (segment (start 88.915 78.73) (end 88.915 74.945) (width 0.25) (layer "F.Cu") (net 14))
 (segment (start 88.915 74.945) (end 88.9 74.93) (width 0.25) (layer "F.Cu") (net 14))
 (segment (start 81.295 78.73) (end 81.295 74.945) (width 0.25) (layer "F.Cu") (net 3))
 (segment (start 81.295 74.945) (end 81.28 74.93) (width 0.25) (layer "F.Cu") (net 3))
 (segment (start 81.28 90.17) (end 81.28 86.365) (width 0.25) (layer "F.Cu") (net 10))
 (segment (start 81.28 86.365) (end 81.295 86.35) (width 0.25) (layer "F.Cu") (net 10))
 (segment (start 88.9 86.365) (end 88.915 86.35) (width 0.25) (layer "F.Cu") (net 4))
 (segment (start 88.9 90.17) (end 88.9 86.365) (width 0.25) (layer "F.Cu") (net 4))
 (segment (start 74.32 91.44) (end 71.12 91.44) (width 0.25) (layer "B.Cu") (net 5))
 (segment (start 88.75 105.87) (end 74.32 91.44) (width 0.25) (layer "B.Cu") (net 5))
 (segment (start 73.74 86.36) (end 71.12 86.36) (width 0.25) (layer "B.Cu") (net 6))
 (segment (start 88.75 101.37) (end 73.74 86.36) (width 0.25) (layer "B.Cu") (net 6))
 (segment (start 73.965991 72.295) (end 69.945 72.295) (width 0.25) (layer "B.Cu") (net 15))
 (segment (start 69.85 72.2) (end 69.85 69.85) (width 0.25) (layer "B.Cu") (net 15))
 (segment (start 78.755 77.084009) (end 73.965991 72.295) (width 0.25) (layer "B.Cu") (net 15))
 (segment (start 69.945 72.295) (end 69.85 72.2) (width 0.25) (layer "B.Cu") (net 15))
 (segment (start 69.85 69.85) (end 71.12 68.58) (width 0.25) (layer "B.Cu") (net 15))
 (segment (start 78.755 78.73) (end 78.755 77.084009) (width 0.25) (layer "B.Cu") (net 15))
 (segment (start 90.33 77.605) (end 79.912387 77.605) (width 0.25) (layer "B.Cu") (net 13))
 (segment (start 79.912387 77.605) (end 73.427387 71.12) (width 0.25) (layer "B.Cu") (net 13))
 (segment (start 73.427387 71.12) (end 71.12 71.12) (width 0.25) (layer "B.Cu") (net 13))
 (segment (start 91.455 78.73) (end 90.33 77.605) (width 0.25) (layer "B.Cu") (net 13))
 (segment (start 77.92 80.5655) (end 77.91 80.5555) (width 0.25) (layer "F.Cu") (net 11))
 (segment (start 77.92 82.0045) (end 77.92 80.5655) (width 0.25) (layer "F.Cu") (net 11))
 (via (at 77.92 82.0045) (size 0.8) (drill 0.4) (layers "F.Cu" "B.Cu") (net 11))
 (via (at 77.91 80.5555) (size 0.8) (drill 0.4) (layers "F.Cu" "B.Cu") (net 11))
 (segment (start 87.1095 82.0045) (end 77.92 82.0045) (width 0.25) (layer "B.Cu") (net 11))
 (segment (start 74.095 77.565) (end 72.73 76.2) (width 0.25) (layer "B.Cu") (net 11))
 (segment (start 91.455 86.35) (end 87.1095 82.0045) (width 0.25) (layer "B.Cu") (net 11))
 (segment (start 76.449509 80.5555) (end 74.095 78.200991) (width 0.25) (layer "B.Cu") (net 11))
 (segment (start 77.91 80.5555) (end 76.449509 80.5555) (width 0.25) (layer "B.Cu") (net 11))
 (segment (start 74.095 78.200991) (end 74.095 77.565) (width 0.25) (layer "B.Cu") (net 11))
 (segment (start 72.73 76.2) (end 71.12 76.2) (width 0.25) (layer "B.Cu") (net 11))
 (segment (start 74.86 82.455) (end 78.755 86.35) (width 0.25) (layer "B.Cu") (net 9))
 (segment (start 69.945 79.915) (end 69.945 82.455) (width 0.25) (layer "B.Cu") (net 9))
 (segment (start 71.12 78.74) (end 69.945 79.915) (width 0.25) (layer "B.Cu") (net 9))
 (segment (start 69.945 82.455) (end 74.86 82.455) (width 0.25) (layer "B.Cu") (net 9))
 (segment (start 91.445 81.28) (end 93.995 78.73) (width 0.25) (layer "B.Cu") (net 12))
 (segment (start 71.12 81.28) (end 91.445 81.28) (width 0.25) (layer "B.Cu") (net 12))
 (segment (start 76.215 86.35) (end 73.685 83.82) (width 0.25) (layer "B.Cu") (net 8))
 (segment (start 73.685 83.82) (end 71.12 83.82) (width 0.25) (layer "B.Cu") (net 8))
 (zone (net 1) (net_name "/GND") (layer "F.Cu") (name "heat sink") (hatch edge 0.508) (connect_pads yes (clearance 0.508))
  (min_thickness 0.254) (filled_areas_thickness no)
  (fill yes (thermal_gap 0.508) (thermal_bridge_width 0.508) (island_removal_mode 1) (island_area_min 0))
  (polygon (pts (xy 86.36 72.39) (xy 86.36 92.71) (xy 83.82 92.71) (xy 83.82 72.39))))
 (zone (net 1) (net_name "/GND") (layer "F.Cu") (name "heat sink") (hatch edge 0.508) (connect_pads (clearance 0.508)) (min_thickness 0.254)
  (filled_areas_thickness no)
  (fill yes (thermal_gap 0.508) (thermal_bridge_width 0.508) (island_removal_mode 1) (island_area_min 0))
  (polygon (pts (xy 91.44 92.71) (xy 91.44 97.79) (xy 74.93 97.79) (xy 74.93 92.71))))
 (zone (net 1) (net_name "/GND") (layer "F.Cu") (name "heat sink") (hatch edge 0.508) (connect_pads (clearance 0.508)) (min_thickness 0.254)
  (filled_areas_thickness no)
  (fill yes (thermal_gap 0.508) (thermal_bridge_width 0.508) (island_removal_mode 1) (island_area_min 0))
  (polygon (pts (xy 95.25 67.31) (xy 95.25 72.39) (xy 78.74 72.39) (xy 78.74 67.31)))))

